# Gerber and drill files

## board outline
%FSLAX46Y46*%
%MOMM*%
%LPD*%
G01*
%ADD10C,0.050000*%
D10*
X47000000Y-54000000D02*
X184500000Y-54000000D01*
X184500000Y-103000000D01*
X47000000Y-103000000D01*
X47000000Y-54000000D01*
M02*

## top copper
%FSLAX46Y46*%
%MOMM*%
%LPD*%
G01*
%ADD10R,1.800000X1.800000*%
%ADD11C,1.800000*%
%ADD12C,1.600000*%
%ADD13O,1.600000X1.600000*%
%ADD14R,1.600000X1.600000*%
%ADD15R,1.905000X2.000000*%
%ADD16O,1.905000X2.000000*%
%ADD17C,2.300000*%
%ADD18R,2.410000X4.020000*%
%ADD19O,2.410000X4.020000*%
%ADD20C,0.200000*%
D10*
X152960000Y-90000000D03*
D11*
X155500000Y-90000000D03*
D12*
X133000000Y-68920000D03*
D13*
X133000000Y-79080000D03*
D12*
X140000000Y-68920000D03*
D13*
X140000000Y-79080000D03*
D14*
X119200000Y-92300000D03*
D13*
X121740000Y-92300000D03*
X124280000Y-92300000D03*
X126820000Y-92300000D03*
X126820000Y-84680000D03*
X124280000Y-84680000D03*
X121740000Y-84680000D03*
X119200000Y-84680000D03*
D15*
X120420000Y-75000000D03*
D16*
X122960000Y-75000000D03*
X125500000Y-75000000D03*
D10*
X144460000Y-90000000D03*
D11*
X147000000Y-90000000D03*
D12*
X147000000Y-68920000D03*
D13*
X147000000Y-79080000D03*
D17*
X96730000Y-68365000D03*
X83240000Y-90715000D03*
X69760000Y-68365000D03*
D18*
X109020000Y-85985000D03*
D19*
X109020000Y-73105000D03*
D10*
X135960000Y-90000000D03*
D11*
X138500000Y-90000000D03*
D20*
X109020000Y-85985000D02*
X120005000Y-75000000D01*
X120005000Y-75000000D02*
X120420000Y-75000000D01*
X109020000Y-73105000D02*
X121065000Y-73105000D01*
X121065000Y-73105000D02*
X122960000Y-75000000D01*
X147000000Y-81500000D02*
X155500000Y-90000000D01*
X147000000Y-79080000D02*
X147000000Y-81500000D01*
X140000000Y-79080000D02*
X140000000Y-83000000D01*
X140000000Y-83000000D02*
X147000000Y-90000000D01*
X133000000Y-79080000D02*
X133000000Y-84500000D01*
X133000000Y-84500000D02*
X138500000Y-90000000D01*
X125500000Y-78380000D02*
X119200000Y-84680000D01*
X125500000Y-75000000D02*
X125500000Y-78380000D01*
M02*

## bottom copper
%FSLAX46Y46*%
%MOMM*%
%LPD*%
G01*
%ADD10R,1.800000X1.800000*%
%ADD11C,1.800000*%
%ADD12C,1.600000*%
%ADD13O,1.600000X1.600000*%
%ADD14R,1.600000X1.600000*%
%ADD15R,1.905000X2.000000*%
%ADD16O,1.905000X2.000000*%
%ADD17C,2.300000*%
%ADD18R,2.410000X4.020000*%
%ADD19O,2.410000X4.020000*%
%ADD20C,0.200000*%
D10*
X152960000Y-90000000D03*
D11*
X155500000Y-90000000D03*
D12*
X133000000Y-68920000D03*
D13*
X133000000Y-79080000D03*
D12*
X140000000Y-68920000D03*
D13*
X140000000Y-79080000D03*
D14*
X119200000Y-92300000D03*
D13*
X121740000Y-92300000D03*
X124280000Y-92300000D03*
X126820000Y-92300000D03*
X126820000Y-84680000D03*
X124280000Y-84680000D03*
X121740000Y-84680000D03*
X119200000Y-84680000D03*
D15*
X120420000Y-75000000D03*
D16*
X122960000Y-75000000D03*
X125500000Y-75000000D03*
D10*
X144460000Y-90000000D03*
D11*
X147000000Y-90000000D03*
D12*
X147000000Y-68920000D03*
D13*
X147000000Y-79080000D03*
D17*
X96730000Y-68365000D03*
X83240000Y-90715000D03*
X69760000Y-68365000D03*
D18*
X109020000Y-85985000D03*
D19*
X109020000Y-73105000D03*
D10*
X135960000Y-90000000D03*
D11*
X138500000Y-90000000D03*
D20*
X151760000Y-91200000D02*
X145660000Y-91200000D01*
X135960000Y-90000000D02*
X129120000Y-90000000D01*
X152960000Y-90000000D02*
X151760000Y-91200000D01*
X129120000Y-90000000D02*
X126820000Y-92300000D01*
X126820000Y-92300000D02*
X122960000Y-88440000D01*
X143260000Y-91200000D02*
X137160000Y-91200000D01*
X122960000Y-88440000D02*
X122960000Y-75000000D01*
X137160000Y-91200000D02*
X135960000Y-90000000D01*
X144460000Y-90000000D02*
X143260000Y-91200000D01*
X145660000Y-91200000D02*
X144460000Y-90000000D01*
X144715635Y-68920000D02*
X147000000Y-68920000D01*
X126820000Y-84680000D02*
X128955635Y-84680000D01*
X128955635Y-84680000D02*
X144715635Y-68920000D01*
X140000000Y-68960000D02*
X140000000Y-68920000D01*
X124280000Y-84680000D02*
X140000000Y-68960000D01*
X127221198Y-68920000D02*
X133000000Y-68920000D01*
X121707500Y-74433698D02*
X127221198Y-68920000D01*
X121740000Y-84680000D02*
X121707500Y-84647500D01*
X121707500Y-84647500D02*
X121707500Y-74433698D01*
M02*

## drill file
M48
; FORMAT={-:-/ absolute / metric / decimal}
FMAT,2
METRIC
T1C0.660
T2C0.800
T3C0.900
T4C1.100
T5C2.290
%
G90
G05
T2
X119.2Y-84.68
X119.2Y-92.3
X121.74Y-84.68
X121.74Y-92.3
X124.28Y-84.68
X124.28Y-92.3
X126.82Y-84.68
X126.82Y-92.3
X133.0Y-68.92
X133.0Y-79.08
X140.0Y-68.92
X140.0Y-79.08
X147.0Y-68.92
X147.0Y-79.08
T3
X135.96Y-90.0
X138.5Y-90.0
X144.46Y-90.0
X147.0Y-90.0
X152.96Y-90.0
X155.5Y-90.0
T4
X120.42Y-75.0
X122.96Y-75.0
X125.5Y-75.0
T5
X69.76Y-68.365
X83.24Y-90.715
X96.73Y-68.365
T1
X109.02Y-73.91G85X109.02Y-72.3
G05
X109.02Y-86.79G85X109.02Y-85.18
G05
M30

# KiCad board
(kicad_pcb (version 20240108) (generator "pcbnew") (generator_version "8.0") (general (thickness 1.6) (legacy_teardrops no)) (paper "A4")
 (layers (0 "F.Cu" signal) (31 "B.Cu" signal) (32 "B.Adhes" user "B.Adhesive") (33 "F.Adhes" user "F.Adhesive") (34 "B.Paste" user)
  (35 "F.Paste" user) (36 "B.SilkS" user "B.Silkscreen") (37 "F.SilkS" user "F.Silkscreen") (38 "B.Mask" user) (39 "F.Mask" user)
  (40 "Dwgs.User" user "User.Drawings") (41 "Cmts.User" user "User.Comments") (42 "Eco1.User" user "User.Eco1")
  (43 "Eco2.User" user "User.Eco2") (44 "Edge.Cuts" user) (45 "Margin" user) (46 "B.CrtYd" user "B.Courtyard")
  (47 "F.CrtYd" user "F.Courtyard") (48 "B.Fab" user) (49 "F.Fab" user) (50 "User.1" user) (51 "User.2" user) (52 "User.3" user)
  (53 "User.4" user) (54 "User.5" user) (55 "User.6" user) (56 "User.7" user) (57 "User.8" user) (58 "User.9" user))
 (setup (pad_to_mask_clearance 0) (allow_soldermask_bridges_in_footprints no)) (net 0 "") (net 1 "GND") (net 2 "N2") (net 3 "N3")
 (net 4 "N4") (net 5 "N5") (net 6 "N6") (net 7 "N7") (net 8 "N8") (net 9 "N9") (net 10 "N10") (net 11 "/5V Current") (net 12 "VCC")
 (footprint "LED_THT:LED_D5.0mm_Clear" (layer "F.Cu") (at 152.96 90)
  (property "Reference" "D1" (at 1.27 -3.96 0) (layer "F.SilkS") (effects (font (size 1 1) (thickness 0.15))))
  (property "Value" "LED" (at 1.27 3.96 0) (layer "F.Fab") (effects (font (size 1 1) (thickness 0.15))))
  (pad "1" thru_hole rect (at 0 0) (size 1.8 1.8) (drill 0.9) (layers "*.Cu" "*.Mask") (remove_unused_layers no) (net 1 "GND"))
  (pad "2" thru_hole circle (at 2.54 0) (size 1.8 1.8) (drill 0.9) (layers "*.Cu" "*.Mask") (remove_unused_layers no) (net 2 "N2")))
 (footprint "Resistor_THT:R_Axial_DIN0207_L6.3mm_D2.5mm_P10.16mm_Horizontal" (layer "F.Cu") (at 133 68.92 -90)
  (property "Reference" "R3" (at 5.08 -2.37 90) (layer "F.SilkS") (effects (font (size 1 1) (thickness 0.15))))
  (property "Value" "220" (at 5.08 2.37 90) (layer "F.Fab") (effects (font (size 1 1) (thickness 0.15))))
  (pad "1" thru_hole circle (at 0 0 270) (size 1.6 1.6) (drill 0.8) (layers "*.Cu" "*.Mask") (remove_unused_layers no) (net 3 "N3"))
  (pad "2" thru_hole oval (at 10.16 0 270) (size 1.6 1.6) (drill 0.8) (layers "*.Cu" "*.Mask") (remove_unused_layers no) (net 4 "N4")))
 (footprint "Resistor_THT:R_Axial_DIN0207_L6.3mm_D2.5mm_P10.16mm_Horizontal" (layer "F.Cu") (at 140 68.92 -90)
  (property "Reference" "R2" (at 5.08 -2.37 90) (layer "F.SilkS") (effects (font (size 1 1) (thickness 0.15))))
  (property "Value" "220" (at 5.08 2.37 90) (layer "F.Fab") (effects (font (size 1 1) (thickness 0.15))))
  (pad "1" thru_hole circle (at 0 0 270) (size 1.6 1.6) (drill 0.8) (layers "*.Cu" "*.Mask") (remove_unused_layers no) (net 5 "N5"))
  (pad "2" thru_hole oval (at 10.16 0 270) (size 1.6 1.6) (drill 0.8) (layers "*.Cu" "*.Mask") (remove_unused_layers no) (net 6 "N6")))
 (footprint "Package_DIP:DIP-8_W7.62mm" (layer "F.Cu") (at 119.2 92.3 90)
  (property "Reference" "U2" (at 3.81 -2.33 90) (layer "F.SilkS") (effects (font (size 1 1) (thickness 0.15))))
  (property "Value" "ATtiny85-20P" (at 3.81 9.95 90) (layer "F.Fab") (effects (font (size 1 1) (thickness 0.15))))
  (pad "1" thru_hole rect (at 0 0 90) (size 1.6 1.6) (drill 0.8) (layers "*.Cu" "*.Mask") (remove_unused_layers no) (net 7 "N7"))
  (pad "2" thru_hole oval (at 0 2.54 90) (size 1.6 1.6) (drill 0.8) (layers "*.Cu" "*.Mask") (remove_unused_layers no) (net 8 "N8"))
  (pad "3" thru_hole oval (at 0 5.08 90) (size 1.6 1.6) (drill 0.8) (layers "*.Cu" "*.Mask") (remove_unused_layers no) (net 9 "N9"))
  (pad "4" thru_hole oval (at 0 7.62 90) (size 1.6 1.6) (drill 0.8) (layers "*.Cu" "*.Mask") (remove_unused_layers no) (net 1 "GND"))
  (pad "5" thru_hole oval (at 7.62 7.62 90) (size 1.6 1.6) (drill 0.8) (layers "*.Cu" "*.Mask") (remove_unused_layers no) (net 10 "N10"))
  (pad "6" thru_hole oval (at 7.62 5.08 90) (size 1.6 1.6) (drill 0.8) (layers "*.Cu" "*.Mask") (remove_unused_layers no) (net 5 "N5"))
  (pad "7" thru_hole oval (at 7.62 2.54 90) (size 1.6 1.6) (drill 0.8) (layers "*.Cu" "*.Mask") (remove_unused_layers no) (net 3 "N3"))
  (pad "8" thru_hole oval (at 7.62 0 90) (size 1.6 1.6) (drill 0.8) (layers "*.Cu" "*.Mask") (remove_unused_layers no)
   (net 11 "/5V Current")))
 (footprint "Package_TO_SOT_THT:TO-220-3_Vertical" (layer "F.Cu") (at 120.42 75)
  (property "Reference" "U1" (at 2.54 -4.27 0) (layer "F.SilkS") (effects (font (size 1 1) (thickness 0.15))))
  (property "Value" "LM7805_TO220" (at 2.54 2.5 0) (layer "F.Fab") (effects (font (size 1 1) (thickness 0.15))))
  (pad "1" thru_hole rect (at 0 0) (size 1.905 2) (drill 1.1) (layers "*.Cu" "*.Mask") (remove_unused_layers no) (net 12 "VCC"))
  (pad "2" thru_hole oval (at 2.54 0) (size 1.905 2) (drill 1.1) (layers "*.Cu" "*.Mask") (remove_unused_layers no) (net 1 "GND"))
  (pad "3" thru_hole oval (at 5.08 0) (size 1.905 2) (drill 1.1) (layers "*.Cu" "*.Mask") (remove_unused_layers no) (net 11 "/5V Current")))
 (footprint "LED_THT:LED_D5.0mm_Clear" (layer "F.Cu") (at 144.46 90)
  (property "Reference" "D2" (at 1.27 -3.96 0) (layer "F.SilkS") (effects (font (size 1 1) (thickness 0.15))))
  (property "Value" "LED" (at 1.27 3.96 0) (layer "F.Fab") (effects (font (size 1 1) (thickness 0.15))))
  (pad "1" thru_hole rect (at 0 0) (size 1.8 1.8) (drill 0.9) (layers "*.Cu" "*.Mask") (remove_unused_layers no) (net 1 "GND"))
  (pad "2" thru_hole circle (at 2.54 0) (size 1.8 1.8) (drill 0.9) (layers "*.Cu" "*.Mask") (remove_unused_layers no) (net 6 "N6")))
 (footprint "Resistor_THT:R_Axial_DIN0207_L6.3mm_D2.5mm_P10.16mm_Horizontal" (layer "F.Cu") (at 147 68.92 -90)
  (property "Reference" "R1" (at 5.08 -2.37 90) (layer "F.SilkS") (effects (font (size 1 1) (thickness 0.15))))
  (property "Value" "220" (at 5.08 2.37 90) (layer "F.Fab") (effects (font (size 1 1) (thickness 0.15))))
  (pad "1" thru_hole circle (at 0 0 270) (size 1.6 1.6) (drill 0.8) (layers "*.Cu" "*.Mask") (remove_unused_layers no) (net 10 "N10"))
  (pad "2" thru_hole oval (at 10.16 0 270) (size 1.6 1.6) (drill 0.8) (layers "*.Cu" "*.Mask") (remove_unused_layers no) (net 2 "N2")))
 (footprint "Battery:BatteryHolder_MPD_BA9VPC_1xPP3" (layer "F.Cu") (at 109.02 85.985 180)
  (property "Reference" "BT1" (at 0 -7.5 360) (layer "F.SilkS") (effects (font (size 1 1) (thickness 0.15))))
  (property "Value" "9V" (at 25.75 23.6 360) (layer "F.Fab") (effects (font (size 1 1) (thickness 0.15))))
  (pad "" np_thru_hole circle (at 12.29 17.62 180) (size 2.3 2.3) (drill 2.29) (layers "*.Cu" "*.Mask"))
  (pad "" np_thru_hole circle (at 25.78 -4.73 180) (size 2.3 2.3) (drill 2.29) (layers "*.Cu" "*.Mask"))
  (pad "" np_thru_hole circle (at 39.26 17.62 180) (size 2.3 2.3) (drill 2.29) (layers "*.Cu" "*.Mask"))
  (pad "1" thru_hole rect (at 0 0 180) (size 2.41 4.02) (drill oval 0.66 2.27) (layers "*.Cu" "*.Mask") (remove_unused_layers no)
   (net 12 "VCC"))
  (pad "2" thru_hole oval (at 0 12.88 180) (size 2.41 4.02) (drill oval 0.66 2.27) (layers "*.Cu" "*.Mask") (remove_unused_layers no)
   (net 1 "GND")))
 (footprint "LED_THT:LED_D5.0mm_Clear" (layer "F.Cu") (at 135.96 90)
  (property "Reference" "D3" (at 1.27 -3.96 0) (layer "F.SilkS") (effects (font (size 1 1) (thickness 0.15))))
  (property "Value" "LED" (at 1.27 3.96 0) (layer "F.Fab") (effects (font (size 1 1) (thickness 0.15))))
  (pad "1" thru_hole rect (at 0 0) (size 1.8 1.8) (drill 0.9) (layers "*.Cu" "*.Mask") (remove_unused_layers no) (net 1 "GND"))
  (pad "2" thru_hole circle (at 2.54 0) (size 1.8 1.8) (drill 0.9) (layers "*.Cu" "*.Mask") (remove_unused_layers no) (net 4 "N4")))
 (gr_rect (start 47 54) (end 184.5 103) (stroke (width 0.05) (type default)) (fill none) (layer "Edge.Cuts"))
 (segment (start 109.02 85.985) (end 120.005 75) (width 0.2) (layer "F.Cu") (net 12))
 (segment (start 120.005 75) (end 120.42 75) (width 0.2) (layer "F.Cu") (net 12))
 (segment (start 109.02 73.105) (end 121.065 73.105) (width 0.2) (layer "F.Cu") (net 1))
 (segment (start 121.065 73.105) (end 122.96 75) (width 0.2) (layer "F.Cu") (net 1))
 (segment (start 151.76 91.2) (end 145.66 91.2) (width 0.2) (layer "B.Cu") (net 1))
 (segment (start 135.96 90) (end 129.12 90) (width 0.2) (layer "B.Cu") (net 1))
 (segment (start 152.96 90) (end 151.76 91.2) (width 0.2) (layer "B.Cu") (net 1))
 (segment (start 129.12 90) (end 126.82 92.3) (width 0.2) (layer "B.Cu") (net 1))
 (segment (start 126.82 92.3) (end 122.96 88.44) (width 0.2) (layer "B.Cu") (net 1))
 (segment (start 143.26 91.2) (end 137.16 91.2) (width 0.2) (layer "B.Cu") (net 1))
 (segment (start 122.96 88.44) (end 122.96 75) (width 0.2) (layer "B.Cu") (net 1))
 (segment (start 137.16 91.2) (end 135.96 90) (width 0.2) (layer "B.Cu") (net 1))
 (segment (start 144.46 90) (end 143.26 91.2) (width 0.2) (layer "B.Cu") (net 1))
 (segment (start 145.66 91.2) (end 144.46 90) (width 0.2) (layer "B.Cu") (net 1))
 (segment (start 147 81.5) (end 155.5 90) (width 0.2) (layer "F.Cu") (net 2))
 (segment (start 147 79.08) (end 147 81.5) (width 0.2) (layer "F.Cu") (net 2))
 (segment (start 140 79.08) (end 140 83) (width 0.2) (layer "F.Cu") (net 6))
 (segment (start 140 83) (end 147 90) (width 0.2) (layer "F.Cu") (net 6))
 (segment (start 133 79.08) (end 133 84.5) (width 0.2) (layer "F.Cu") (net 4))
 (segment (start 133 84.5) (end 138.5 90) (width 0.2) (layer "F.Cu") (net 4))
 (segment (start 144.715635 68.92) (end 147 68.92) (width 0.2) (layer "B.Cu") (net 10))
 (segment (start 126.82 84.68) (end 128.955635 84.68) (width 0.2) (layer "B.Cu") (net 10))
 (segment (start 128.955635 84.68) (end 144.715635 68.92) (width 0.2) (layer "B.Cu") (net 10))
 (segment (start 140 68.96) (end 140 68.92) (width 0.2) (layer "B.Cu") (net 5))
 (segment (start 124.28 84.68) (end 140 68.96) (width 0.2) (layer "B.Cu") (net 5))
 (segment (start 127.221198 68.92) (end 133 68.92) (width 0.2) (layer "B.Cu") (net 3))
 (segment (start 121.7075 74.433698) (end 127.221198 68.92) (width 0.2) (layer "B.Cu") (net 3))
 (segment (start 121.74 84.68) (end 121.7075 84.6475) (width 0.2) (layer "B.Cu") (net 3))
 (segment (start 121.7075 84.6475) (end 121.7075 74.433698) (width 0.2) (layer "B.Cu") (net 3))
 (segment (start 125.5 78.38) (end 119.2 84.68) (width 0.2) (layer "F.Cu") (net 11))
 (segment (start 125.5 75) (end 125.5 78.38) (width 0.2) (layer "F.Cu") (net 11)))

